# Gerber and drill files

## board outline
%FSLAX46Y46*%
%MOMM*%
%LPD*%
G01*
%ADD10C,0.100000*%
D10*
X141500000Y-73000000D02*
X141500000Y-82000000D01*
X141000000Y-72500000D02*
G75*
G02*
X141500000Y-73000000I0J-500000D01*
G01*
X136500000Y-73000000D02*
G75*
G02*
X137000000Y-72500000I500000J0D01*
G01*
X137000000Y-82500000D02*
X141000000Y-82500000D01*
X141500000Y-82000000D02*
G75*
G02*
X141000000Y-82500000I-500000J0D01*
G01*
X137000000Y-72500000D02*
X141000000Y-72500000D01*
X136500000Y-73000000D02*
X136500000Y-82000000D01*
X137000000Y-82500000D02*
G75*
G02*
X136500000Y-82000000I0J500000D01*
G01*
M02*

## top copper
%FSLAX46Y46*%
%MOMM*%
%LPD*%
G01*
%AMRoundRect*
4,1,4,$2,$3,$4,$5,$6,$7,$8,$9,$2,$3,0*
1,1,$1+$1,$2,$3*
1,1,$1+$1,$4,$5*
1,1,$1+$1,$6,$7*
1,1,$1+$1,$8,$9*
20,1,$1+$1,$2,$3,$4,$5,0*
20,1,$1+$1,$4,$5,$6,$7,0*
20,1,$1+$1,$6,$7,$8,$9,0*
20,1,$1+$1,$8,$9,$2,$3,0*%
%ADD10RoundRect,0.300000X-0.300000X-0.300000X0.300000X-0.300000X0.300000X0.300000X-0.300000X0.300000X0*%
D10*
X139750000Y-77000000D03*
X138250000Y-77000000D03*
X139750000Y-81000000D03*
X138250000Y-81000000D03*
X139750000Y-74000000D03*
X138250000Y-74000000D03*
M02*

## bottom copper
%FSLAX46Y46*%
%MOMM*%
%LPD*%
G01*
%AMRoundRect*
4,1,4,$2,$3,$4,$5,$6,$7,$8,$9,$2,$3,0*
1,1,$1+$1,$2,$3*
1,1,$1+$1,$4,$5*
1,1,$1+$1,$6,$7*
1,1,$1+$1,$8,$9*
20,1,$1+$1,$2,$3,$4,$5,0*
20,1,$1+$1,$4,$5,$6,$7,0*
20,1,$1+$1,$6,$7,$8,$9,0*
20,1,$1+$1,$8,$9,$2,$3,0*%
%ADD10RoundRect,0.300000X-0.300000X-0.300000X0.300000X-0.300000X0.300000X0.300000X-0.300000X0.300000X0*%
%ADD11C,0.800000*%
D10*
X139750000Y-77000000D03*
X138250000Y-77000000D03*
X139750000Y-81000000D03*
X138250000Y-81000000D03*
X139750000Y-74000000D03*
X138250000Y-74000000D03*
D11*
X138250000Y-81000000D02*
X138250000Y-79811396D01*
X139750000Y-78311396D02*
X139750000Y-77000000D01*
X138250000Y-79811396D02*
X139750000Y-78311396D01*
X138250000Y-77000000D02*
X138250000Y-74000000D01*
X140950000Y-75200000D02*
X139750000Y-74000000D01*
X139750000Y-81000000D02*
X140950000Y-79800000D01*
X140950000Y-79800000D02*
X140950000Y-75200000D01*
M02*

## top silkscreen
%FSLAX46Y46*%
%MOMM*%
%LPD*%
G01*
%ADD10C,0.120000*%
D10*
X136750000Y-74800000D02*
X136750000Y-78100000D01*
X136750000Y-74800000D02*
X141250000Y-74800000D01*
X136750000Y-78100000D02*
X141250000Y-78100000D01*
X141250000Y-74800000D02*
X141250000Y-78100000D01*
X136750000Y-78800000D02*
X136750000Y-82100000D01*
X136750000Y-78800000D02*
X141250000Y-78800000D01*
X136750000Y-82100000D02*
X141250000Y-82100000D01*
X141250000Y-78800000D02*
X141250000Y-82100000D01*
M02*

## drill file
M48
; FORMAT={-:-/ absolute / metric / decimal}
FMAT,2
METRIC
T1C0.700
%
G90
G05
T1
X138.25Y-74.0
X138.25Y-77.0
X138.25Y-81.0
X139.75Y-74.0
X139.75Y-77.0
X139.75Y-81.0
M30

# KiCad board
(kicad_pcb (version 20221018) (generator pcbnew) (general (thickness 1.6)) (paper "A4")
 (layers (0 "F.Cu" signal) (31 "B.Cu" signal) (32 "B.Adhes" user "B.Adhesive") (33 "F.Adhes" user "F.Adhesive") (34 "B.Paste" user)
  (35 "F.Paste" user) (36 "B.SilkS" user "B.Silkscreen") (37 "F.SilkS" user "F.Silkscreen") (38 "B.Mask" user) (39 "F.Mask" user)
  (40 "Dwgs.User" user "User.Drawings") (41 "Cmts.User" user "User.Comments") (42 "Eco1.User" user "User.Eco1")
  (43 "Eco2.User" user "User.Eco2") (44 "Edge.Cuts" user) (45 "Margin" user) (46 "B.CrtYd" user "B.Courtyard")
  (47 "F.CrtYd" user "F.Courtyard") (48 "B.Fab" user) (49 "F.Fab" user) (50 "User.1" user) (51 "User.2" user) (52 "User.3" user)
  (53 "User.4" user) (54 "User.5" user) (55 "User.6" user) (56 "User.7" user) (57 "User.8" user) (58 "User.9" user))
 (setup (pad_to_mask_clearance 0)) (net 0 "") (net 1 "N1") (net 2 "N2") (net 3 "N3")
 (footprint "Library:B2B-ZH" (layer "F.Cu") (at 139 77)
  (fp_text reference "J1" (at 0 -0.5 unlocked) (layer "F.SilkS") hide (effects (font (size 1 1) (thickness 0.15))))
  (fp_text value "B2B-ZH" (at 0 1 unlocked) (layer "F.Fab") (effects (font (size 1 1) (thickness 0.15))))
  (fp_line (start -2.25 -2.2) (end -2.25 1.1) (stroke (width 0.12) (type default)) (layer "F.SilkS"))
  (fp_line (start -2.25 -2.2) (end 2.25 -2.2) (stroke (width 0.12) (type default)) (layer "F.SilkS"))
  (fp_line (start -2.25 1.1) (end 2.25 1.1) (stroke (width 0.12) (type default)) (layer "F.SilkS"))
  (fp_line (start 2.25 -2.2) (end 2.25 1.1) (stroke (width 0.12) (type default)) (layer "F.SilkS"))
  (pad "1" thru_hole roundrect (at 0.75 0) (size 1.2 1.2) (drill 0.7) (layers "*.Cu" "*.Mask") (roundrect_rratio 0.25) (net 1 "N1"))
  (pad "2" thru_hole roundrect (at -0.75 0) (size 1.2 1.2) (drill 0.7) (layers "*.Cu" "*.Mask") (roundrect_rratio 0.25) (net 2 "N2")))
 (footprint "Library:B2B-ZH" (layer "F.Cu") (at 139 81)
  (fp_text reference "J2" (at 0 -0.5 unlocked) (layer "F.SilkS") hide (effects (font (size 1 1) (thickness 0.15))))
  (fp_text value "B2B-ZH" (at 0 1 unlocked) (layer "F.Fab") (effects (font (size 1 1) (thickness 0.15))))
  (fp_line (start -2.25 -2.2) (end -2.25 1.1) (stroke (width 0.12) (type default)) (layer "F.SilkS"))
  (fp_line (start -2.25 -2.2) (end 2.25 -2.2) (stroke (width 0.12) (type default)) (layer "F.SilkS"))
  (fp_line (start -2.25 1.1) (end 2.25 1.1) (stroke (width 0.12) (type default)) (layer "F.SilkS"))
  (fp_line (start 2.25 -2.2) (end 2.25 1.1) (stroke (width 0.12) (type default)) (layer "F.SilkS"))
  (pad "1" thru_hole roundrect (at 0.75 0) (size 1.2 1.2) (drill 0.7) (layers "*.Cu" "*.Mask") (roundrect_rratio 0.25) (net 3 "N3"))
  (pad "2" thru_hole roundrect (at -0.75 0) (size 1.2 1.2) (drill 0.7) (layers "*.Cu" "*.Mask") (roundrect_rratio 0.25) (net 1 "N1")))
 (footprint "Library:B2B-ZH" (layer "B.Cu") (at 139 74)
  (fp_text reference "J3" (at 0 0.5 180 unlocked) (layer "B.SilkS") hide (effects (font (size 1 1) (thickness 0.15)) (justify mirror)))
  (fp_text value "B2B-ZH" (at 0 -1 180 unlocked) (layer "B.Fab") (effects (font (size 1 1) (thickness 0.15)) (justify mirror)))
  (pad "1" thru_hole roundrect (at 0.75 0) (size 1.2 1.2) (drill 0.7) (layers "*.Cu" "*.Mask") (roundrect_rratio 0.25) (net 3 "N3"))
  (pad "2" thru_hole roundrect (at -0.75 0) (size 1.2 1.2) (drill 0.7) (layers "*.Cu" "*.Mask") (roundrect_rratio 0.25) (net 2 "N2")))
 (gr_line (start 141.5 73) (end 141.5 82) (stroke (width 0.1) (type default)) (layer "Edge.Cuts"))
 (gr_arc (start 141 72.5) (mid 141.353553 72.646447) (end 141.5 73) (stroke (width 0.1) (type default)) (layer "Edge.Cuts"))
 (gr_arc (start 136.5 73) (mid 136.646447 72.646447) (end 137 72.5) (stroke (width 0.1) (type default)) (layer "Edge.Cuts"))
 (gr_line (start 137 82.5) (end 141 82.5) (stroke (width 0.1) (type default)) (layer "Edge.Cuts"))
 (gr_arc (start 141.5 82) (mid 141.353553 82.353553) (end 141 82.5) (stroke (width 0.1) (type default)) (layer "Edge.Cuts"))
 (gr_line (start 137 72.5) (end 141 72.5) (stroke (width 0.1) (type default)) (layer "Edge.Cuts"))
 (gr_line (start 136.5 73) (end 136.5 82) (stroke (width 0.1) (type default)) (layer "Edge.Cuts"))
 (gr_arc (start 137 82.5) (mid 136.646447 82.353553) (end 136.5 82) (stroke (width 0.1) (type default)) (layer "Edge.Cuts"))
 (segment (start 138.25 81) (end 138.25 79.811396) (width 0.8) (layer "B.Cu") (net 1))
 (segment (start 139.75 78.311396) (end 139.75 77) (width 0.8) (layer "B.Cu") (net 1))
 (segment (start 138.25 79.811396) (end 139.75 78.311396) (width 0.8) (layer "B.Cu") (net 1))
 (segment (start 138.25 77) (end 138.25 74) (width 0.8) (layer "B.Cu") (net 2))
 (segment (start 140.95 75.2) (end 139.75 74) (width 0.8) (layer "B.Cu") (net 3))
 (segment (start 139.75 81) (end 140.95 79.8) (width 0.8) (layer "B.Cu") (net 3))
 (segment (start 140.95 79.8) (end 140.95 75.2) (width 0.8) (layer "B.Cu") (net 3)))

